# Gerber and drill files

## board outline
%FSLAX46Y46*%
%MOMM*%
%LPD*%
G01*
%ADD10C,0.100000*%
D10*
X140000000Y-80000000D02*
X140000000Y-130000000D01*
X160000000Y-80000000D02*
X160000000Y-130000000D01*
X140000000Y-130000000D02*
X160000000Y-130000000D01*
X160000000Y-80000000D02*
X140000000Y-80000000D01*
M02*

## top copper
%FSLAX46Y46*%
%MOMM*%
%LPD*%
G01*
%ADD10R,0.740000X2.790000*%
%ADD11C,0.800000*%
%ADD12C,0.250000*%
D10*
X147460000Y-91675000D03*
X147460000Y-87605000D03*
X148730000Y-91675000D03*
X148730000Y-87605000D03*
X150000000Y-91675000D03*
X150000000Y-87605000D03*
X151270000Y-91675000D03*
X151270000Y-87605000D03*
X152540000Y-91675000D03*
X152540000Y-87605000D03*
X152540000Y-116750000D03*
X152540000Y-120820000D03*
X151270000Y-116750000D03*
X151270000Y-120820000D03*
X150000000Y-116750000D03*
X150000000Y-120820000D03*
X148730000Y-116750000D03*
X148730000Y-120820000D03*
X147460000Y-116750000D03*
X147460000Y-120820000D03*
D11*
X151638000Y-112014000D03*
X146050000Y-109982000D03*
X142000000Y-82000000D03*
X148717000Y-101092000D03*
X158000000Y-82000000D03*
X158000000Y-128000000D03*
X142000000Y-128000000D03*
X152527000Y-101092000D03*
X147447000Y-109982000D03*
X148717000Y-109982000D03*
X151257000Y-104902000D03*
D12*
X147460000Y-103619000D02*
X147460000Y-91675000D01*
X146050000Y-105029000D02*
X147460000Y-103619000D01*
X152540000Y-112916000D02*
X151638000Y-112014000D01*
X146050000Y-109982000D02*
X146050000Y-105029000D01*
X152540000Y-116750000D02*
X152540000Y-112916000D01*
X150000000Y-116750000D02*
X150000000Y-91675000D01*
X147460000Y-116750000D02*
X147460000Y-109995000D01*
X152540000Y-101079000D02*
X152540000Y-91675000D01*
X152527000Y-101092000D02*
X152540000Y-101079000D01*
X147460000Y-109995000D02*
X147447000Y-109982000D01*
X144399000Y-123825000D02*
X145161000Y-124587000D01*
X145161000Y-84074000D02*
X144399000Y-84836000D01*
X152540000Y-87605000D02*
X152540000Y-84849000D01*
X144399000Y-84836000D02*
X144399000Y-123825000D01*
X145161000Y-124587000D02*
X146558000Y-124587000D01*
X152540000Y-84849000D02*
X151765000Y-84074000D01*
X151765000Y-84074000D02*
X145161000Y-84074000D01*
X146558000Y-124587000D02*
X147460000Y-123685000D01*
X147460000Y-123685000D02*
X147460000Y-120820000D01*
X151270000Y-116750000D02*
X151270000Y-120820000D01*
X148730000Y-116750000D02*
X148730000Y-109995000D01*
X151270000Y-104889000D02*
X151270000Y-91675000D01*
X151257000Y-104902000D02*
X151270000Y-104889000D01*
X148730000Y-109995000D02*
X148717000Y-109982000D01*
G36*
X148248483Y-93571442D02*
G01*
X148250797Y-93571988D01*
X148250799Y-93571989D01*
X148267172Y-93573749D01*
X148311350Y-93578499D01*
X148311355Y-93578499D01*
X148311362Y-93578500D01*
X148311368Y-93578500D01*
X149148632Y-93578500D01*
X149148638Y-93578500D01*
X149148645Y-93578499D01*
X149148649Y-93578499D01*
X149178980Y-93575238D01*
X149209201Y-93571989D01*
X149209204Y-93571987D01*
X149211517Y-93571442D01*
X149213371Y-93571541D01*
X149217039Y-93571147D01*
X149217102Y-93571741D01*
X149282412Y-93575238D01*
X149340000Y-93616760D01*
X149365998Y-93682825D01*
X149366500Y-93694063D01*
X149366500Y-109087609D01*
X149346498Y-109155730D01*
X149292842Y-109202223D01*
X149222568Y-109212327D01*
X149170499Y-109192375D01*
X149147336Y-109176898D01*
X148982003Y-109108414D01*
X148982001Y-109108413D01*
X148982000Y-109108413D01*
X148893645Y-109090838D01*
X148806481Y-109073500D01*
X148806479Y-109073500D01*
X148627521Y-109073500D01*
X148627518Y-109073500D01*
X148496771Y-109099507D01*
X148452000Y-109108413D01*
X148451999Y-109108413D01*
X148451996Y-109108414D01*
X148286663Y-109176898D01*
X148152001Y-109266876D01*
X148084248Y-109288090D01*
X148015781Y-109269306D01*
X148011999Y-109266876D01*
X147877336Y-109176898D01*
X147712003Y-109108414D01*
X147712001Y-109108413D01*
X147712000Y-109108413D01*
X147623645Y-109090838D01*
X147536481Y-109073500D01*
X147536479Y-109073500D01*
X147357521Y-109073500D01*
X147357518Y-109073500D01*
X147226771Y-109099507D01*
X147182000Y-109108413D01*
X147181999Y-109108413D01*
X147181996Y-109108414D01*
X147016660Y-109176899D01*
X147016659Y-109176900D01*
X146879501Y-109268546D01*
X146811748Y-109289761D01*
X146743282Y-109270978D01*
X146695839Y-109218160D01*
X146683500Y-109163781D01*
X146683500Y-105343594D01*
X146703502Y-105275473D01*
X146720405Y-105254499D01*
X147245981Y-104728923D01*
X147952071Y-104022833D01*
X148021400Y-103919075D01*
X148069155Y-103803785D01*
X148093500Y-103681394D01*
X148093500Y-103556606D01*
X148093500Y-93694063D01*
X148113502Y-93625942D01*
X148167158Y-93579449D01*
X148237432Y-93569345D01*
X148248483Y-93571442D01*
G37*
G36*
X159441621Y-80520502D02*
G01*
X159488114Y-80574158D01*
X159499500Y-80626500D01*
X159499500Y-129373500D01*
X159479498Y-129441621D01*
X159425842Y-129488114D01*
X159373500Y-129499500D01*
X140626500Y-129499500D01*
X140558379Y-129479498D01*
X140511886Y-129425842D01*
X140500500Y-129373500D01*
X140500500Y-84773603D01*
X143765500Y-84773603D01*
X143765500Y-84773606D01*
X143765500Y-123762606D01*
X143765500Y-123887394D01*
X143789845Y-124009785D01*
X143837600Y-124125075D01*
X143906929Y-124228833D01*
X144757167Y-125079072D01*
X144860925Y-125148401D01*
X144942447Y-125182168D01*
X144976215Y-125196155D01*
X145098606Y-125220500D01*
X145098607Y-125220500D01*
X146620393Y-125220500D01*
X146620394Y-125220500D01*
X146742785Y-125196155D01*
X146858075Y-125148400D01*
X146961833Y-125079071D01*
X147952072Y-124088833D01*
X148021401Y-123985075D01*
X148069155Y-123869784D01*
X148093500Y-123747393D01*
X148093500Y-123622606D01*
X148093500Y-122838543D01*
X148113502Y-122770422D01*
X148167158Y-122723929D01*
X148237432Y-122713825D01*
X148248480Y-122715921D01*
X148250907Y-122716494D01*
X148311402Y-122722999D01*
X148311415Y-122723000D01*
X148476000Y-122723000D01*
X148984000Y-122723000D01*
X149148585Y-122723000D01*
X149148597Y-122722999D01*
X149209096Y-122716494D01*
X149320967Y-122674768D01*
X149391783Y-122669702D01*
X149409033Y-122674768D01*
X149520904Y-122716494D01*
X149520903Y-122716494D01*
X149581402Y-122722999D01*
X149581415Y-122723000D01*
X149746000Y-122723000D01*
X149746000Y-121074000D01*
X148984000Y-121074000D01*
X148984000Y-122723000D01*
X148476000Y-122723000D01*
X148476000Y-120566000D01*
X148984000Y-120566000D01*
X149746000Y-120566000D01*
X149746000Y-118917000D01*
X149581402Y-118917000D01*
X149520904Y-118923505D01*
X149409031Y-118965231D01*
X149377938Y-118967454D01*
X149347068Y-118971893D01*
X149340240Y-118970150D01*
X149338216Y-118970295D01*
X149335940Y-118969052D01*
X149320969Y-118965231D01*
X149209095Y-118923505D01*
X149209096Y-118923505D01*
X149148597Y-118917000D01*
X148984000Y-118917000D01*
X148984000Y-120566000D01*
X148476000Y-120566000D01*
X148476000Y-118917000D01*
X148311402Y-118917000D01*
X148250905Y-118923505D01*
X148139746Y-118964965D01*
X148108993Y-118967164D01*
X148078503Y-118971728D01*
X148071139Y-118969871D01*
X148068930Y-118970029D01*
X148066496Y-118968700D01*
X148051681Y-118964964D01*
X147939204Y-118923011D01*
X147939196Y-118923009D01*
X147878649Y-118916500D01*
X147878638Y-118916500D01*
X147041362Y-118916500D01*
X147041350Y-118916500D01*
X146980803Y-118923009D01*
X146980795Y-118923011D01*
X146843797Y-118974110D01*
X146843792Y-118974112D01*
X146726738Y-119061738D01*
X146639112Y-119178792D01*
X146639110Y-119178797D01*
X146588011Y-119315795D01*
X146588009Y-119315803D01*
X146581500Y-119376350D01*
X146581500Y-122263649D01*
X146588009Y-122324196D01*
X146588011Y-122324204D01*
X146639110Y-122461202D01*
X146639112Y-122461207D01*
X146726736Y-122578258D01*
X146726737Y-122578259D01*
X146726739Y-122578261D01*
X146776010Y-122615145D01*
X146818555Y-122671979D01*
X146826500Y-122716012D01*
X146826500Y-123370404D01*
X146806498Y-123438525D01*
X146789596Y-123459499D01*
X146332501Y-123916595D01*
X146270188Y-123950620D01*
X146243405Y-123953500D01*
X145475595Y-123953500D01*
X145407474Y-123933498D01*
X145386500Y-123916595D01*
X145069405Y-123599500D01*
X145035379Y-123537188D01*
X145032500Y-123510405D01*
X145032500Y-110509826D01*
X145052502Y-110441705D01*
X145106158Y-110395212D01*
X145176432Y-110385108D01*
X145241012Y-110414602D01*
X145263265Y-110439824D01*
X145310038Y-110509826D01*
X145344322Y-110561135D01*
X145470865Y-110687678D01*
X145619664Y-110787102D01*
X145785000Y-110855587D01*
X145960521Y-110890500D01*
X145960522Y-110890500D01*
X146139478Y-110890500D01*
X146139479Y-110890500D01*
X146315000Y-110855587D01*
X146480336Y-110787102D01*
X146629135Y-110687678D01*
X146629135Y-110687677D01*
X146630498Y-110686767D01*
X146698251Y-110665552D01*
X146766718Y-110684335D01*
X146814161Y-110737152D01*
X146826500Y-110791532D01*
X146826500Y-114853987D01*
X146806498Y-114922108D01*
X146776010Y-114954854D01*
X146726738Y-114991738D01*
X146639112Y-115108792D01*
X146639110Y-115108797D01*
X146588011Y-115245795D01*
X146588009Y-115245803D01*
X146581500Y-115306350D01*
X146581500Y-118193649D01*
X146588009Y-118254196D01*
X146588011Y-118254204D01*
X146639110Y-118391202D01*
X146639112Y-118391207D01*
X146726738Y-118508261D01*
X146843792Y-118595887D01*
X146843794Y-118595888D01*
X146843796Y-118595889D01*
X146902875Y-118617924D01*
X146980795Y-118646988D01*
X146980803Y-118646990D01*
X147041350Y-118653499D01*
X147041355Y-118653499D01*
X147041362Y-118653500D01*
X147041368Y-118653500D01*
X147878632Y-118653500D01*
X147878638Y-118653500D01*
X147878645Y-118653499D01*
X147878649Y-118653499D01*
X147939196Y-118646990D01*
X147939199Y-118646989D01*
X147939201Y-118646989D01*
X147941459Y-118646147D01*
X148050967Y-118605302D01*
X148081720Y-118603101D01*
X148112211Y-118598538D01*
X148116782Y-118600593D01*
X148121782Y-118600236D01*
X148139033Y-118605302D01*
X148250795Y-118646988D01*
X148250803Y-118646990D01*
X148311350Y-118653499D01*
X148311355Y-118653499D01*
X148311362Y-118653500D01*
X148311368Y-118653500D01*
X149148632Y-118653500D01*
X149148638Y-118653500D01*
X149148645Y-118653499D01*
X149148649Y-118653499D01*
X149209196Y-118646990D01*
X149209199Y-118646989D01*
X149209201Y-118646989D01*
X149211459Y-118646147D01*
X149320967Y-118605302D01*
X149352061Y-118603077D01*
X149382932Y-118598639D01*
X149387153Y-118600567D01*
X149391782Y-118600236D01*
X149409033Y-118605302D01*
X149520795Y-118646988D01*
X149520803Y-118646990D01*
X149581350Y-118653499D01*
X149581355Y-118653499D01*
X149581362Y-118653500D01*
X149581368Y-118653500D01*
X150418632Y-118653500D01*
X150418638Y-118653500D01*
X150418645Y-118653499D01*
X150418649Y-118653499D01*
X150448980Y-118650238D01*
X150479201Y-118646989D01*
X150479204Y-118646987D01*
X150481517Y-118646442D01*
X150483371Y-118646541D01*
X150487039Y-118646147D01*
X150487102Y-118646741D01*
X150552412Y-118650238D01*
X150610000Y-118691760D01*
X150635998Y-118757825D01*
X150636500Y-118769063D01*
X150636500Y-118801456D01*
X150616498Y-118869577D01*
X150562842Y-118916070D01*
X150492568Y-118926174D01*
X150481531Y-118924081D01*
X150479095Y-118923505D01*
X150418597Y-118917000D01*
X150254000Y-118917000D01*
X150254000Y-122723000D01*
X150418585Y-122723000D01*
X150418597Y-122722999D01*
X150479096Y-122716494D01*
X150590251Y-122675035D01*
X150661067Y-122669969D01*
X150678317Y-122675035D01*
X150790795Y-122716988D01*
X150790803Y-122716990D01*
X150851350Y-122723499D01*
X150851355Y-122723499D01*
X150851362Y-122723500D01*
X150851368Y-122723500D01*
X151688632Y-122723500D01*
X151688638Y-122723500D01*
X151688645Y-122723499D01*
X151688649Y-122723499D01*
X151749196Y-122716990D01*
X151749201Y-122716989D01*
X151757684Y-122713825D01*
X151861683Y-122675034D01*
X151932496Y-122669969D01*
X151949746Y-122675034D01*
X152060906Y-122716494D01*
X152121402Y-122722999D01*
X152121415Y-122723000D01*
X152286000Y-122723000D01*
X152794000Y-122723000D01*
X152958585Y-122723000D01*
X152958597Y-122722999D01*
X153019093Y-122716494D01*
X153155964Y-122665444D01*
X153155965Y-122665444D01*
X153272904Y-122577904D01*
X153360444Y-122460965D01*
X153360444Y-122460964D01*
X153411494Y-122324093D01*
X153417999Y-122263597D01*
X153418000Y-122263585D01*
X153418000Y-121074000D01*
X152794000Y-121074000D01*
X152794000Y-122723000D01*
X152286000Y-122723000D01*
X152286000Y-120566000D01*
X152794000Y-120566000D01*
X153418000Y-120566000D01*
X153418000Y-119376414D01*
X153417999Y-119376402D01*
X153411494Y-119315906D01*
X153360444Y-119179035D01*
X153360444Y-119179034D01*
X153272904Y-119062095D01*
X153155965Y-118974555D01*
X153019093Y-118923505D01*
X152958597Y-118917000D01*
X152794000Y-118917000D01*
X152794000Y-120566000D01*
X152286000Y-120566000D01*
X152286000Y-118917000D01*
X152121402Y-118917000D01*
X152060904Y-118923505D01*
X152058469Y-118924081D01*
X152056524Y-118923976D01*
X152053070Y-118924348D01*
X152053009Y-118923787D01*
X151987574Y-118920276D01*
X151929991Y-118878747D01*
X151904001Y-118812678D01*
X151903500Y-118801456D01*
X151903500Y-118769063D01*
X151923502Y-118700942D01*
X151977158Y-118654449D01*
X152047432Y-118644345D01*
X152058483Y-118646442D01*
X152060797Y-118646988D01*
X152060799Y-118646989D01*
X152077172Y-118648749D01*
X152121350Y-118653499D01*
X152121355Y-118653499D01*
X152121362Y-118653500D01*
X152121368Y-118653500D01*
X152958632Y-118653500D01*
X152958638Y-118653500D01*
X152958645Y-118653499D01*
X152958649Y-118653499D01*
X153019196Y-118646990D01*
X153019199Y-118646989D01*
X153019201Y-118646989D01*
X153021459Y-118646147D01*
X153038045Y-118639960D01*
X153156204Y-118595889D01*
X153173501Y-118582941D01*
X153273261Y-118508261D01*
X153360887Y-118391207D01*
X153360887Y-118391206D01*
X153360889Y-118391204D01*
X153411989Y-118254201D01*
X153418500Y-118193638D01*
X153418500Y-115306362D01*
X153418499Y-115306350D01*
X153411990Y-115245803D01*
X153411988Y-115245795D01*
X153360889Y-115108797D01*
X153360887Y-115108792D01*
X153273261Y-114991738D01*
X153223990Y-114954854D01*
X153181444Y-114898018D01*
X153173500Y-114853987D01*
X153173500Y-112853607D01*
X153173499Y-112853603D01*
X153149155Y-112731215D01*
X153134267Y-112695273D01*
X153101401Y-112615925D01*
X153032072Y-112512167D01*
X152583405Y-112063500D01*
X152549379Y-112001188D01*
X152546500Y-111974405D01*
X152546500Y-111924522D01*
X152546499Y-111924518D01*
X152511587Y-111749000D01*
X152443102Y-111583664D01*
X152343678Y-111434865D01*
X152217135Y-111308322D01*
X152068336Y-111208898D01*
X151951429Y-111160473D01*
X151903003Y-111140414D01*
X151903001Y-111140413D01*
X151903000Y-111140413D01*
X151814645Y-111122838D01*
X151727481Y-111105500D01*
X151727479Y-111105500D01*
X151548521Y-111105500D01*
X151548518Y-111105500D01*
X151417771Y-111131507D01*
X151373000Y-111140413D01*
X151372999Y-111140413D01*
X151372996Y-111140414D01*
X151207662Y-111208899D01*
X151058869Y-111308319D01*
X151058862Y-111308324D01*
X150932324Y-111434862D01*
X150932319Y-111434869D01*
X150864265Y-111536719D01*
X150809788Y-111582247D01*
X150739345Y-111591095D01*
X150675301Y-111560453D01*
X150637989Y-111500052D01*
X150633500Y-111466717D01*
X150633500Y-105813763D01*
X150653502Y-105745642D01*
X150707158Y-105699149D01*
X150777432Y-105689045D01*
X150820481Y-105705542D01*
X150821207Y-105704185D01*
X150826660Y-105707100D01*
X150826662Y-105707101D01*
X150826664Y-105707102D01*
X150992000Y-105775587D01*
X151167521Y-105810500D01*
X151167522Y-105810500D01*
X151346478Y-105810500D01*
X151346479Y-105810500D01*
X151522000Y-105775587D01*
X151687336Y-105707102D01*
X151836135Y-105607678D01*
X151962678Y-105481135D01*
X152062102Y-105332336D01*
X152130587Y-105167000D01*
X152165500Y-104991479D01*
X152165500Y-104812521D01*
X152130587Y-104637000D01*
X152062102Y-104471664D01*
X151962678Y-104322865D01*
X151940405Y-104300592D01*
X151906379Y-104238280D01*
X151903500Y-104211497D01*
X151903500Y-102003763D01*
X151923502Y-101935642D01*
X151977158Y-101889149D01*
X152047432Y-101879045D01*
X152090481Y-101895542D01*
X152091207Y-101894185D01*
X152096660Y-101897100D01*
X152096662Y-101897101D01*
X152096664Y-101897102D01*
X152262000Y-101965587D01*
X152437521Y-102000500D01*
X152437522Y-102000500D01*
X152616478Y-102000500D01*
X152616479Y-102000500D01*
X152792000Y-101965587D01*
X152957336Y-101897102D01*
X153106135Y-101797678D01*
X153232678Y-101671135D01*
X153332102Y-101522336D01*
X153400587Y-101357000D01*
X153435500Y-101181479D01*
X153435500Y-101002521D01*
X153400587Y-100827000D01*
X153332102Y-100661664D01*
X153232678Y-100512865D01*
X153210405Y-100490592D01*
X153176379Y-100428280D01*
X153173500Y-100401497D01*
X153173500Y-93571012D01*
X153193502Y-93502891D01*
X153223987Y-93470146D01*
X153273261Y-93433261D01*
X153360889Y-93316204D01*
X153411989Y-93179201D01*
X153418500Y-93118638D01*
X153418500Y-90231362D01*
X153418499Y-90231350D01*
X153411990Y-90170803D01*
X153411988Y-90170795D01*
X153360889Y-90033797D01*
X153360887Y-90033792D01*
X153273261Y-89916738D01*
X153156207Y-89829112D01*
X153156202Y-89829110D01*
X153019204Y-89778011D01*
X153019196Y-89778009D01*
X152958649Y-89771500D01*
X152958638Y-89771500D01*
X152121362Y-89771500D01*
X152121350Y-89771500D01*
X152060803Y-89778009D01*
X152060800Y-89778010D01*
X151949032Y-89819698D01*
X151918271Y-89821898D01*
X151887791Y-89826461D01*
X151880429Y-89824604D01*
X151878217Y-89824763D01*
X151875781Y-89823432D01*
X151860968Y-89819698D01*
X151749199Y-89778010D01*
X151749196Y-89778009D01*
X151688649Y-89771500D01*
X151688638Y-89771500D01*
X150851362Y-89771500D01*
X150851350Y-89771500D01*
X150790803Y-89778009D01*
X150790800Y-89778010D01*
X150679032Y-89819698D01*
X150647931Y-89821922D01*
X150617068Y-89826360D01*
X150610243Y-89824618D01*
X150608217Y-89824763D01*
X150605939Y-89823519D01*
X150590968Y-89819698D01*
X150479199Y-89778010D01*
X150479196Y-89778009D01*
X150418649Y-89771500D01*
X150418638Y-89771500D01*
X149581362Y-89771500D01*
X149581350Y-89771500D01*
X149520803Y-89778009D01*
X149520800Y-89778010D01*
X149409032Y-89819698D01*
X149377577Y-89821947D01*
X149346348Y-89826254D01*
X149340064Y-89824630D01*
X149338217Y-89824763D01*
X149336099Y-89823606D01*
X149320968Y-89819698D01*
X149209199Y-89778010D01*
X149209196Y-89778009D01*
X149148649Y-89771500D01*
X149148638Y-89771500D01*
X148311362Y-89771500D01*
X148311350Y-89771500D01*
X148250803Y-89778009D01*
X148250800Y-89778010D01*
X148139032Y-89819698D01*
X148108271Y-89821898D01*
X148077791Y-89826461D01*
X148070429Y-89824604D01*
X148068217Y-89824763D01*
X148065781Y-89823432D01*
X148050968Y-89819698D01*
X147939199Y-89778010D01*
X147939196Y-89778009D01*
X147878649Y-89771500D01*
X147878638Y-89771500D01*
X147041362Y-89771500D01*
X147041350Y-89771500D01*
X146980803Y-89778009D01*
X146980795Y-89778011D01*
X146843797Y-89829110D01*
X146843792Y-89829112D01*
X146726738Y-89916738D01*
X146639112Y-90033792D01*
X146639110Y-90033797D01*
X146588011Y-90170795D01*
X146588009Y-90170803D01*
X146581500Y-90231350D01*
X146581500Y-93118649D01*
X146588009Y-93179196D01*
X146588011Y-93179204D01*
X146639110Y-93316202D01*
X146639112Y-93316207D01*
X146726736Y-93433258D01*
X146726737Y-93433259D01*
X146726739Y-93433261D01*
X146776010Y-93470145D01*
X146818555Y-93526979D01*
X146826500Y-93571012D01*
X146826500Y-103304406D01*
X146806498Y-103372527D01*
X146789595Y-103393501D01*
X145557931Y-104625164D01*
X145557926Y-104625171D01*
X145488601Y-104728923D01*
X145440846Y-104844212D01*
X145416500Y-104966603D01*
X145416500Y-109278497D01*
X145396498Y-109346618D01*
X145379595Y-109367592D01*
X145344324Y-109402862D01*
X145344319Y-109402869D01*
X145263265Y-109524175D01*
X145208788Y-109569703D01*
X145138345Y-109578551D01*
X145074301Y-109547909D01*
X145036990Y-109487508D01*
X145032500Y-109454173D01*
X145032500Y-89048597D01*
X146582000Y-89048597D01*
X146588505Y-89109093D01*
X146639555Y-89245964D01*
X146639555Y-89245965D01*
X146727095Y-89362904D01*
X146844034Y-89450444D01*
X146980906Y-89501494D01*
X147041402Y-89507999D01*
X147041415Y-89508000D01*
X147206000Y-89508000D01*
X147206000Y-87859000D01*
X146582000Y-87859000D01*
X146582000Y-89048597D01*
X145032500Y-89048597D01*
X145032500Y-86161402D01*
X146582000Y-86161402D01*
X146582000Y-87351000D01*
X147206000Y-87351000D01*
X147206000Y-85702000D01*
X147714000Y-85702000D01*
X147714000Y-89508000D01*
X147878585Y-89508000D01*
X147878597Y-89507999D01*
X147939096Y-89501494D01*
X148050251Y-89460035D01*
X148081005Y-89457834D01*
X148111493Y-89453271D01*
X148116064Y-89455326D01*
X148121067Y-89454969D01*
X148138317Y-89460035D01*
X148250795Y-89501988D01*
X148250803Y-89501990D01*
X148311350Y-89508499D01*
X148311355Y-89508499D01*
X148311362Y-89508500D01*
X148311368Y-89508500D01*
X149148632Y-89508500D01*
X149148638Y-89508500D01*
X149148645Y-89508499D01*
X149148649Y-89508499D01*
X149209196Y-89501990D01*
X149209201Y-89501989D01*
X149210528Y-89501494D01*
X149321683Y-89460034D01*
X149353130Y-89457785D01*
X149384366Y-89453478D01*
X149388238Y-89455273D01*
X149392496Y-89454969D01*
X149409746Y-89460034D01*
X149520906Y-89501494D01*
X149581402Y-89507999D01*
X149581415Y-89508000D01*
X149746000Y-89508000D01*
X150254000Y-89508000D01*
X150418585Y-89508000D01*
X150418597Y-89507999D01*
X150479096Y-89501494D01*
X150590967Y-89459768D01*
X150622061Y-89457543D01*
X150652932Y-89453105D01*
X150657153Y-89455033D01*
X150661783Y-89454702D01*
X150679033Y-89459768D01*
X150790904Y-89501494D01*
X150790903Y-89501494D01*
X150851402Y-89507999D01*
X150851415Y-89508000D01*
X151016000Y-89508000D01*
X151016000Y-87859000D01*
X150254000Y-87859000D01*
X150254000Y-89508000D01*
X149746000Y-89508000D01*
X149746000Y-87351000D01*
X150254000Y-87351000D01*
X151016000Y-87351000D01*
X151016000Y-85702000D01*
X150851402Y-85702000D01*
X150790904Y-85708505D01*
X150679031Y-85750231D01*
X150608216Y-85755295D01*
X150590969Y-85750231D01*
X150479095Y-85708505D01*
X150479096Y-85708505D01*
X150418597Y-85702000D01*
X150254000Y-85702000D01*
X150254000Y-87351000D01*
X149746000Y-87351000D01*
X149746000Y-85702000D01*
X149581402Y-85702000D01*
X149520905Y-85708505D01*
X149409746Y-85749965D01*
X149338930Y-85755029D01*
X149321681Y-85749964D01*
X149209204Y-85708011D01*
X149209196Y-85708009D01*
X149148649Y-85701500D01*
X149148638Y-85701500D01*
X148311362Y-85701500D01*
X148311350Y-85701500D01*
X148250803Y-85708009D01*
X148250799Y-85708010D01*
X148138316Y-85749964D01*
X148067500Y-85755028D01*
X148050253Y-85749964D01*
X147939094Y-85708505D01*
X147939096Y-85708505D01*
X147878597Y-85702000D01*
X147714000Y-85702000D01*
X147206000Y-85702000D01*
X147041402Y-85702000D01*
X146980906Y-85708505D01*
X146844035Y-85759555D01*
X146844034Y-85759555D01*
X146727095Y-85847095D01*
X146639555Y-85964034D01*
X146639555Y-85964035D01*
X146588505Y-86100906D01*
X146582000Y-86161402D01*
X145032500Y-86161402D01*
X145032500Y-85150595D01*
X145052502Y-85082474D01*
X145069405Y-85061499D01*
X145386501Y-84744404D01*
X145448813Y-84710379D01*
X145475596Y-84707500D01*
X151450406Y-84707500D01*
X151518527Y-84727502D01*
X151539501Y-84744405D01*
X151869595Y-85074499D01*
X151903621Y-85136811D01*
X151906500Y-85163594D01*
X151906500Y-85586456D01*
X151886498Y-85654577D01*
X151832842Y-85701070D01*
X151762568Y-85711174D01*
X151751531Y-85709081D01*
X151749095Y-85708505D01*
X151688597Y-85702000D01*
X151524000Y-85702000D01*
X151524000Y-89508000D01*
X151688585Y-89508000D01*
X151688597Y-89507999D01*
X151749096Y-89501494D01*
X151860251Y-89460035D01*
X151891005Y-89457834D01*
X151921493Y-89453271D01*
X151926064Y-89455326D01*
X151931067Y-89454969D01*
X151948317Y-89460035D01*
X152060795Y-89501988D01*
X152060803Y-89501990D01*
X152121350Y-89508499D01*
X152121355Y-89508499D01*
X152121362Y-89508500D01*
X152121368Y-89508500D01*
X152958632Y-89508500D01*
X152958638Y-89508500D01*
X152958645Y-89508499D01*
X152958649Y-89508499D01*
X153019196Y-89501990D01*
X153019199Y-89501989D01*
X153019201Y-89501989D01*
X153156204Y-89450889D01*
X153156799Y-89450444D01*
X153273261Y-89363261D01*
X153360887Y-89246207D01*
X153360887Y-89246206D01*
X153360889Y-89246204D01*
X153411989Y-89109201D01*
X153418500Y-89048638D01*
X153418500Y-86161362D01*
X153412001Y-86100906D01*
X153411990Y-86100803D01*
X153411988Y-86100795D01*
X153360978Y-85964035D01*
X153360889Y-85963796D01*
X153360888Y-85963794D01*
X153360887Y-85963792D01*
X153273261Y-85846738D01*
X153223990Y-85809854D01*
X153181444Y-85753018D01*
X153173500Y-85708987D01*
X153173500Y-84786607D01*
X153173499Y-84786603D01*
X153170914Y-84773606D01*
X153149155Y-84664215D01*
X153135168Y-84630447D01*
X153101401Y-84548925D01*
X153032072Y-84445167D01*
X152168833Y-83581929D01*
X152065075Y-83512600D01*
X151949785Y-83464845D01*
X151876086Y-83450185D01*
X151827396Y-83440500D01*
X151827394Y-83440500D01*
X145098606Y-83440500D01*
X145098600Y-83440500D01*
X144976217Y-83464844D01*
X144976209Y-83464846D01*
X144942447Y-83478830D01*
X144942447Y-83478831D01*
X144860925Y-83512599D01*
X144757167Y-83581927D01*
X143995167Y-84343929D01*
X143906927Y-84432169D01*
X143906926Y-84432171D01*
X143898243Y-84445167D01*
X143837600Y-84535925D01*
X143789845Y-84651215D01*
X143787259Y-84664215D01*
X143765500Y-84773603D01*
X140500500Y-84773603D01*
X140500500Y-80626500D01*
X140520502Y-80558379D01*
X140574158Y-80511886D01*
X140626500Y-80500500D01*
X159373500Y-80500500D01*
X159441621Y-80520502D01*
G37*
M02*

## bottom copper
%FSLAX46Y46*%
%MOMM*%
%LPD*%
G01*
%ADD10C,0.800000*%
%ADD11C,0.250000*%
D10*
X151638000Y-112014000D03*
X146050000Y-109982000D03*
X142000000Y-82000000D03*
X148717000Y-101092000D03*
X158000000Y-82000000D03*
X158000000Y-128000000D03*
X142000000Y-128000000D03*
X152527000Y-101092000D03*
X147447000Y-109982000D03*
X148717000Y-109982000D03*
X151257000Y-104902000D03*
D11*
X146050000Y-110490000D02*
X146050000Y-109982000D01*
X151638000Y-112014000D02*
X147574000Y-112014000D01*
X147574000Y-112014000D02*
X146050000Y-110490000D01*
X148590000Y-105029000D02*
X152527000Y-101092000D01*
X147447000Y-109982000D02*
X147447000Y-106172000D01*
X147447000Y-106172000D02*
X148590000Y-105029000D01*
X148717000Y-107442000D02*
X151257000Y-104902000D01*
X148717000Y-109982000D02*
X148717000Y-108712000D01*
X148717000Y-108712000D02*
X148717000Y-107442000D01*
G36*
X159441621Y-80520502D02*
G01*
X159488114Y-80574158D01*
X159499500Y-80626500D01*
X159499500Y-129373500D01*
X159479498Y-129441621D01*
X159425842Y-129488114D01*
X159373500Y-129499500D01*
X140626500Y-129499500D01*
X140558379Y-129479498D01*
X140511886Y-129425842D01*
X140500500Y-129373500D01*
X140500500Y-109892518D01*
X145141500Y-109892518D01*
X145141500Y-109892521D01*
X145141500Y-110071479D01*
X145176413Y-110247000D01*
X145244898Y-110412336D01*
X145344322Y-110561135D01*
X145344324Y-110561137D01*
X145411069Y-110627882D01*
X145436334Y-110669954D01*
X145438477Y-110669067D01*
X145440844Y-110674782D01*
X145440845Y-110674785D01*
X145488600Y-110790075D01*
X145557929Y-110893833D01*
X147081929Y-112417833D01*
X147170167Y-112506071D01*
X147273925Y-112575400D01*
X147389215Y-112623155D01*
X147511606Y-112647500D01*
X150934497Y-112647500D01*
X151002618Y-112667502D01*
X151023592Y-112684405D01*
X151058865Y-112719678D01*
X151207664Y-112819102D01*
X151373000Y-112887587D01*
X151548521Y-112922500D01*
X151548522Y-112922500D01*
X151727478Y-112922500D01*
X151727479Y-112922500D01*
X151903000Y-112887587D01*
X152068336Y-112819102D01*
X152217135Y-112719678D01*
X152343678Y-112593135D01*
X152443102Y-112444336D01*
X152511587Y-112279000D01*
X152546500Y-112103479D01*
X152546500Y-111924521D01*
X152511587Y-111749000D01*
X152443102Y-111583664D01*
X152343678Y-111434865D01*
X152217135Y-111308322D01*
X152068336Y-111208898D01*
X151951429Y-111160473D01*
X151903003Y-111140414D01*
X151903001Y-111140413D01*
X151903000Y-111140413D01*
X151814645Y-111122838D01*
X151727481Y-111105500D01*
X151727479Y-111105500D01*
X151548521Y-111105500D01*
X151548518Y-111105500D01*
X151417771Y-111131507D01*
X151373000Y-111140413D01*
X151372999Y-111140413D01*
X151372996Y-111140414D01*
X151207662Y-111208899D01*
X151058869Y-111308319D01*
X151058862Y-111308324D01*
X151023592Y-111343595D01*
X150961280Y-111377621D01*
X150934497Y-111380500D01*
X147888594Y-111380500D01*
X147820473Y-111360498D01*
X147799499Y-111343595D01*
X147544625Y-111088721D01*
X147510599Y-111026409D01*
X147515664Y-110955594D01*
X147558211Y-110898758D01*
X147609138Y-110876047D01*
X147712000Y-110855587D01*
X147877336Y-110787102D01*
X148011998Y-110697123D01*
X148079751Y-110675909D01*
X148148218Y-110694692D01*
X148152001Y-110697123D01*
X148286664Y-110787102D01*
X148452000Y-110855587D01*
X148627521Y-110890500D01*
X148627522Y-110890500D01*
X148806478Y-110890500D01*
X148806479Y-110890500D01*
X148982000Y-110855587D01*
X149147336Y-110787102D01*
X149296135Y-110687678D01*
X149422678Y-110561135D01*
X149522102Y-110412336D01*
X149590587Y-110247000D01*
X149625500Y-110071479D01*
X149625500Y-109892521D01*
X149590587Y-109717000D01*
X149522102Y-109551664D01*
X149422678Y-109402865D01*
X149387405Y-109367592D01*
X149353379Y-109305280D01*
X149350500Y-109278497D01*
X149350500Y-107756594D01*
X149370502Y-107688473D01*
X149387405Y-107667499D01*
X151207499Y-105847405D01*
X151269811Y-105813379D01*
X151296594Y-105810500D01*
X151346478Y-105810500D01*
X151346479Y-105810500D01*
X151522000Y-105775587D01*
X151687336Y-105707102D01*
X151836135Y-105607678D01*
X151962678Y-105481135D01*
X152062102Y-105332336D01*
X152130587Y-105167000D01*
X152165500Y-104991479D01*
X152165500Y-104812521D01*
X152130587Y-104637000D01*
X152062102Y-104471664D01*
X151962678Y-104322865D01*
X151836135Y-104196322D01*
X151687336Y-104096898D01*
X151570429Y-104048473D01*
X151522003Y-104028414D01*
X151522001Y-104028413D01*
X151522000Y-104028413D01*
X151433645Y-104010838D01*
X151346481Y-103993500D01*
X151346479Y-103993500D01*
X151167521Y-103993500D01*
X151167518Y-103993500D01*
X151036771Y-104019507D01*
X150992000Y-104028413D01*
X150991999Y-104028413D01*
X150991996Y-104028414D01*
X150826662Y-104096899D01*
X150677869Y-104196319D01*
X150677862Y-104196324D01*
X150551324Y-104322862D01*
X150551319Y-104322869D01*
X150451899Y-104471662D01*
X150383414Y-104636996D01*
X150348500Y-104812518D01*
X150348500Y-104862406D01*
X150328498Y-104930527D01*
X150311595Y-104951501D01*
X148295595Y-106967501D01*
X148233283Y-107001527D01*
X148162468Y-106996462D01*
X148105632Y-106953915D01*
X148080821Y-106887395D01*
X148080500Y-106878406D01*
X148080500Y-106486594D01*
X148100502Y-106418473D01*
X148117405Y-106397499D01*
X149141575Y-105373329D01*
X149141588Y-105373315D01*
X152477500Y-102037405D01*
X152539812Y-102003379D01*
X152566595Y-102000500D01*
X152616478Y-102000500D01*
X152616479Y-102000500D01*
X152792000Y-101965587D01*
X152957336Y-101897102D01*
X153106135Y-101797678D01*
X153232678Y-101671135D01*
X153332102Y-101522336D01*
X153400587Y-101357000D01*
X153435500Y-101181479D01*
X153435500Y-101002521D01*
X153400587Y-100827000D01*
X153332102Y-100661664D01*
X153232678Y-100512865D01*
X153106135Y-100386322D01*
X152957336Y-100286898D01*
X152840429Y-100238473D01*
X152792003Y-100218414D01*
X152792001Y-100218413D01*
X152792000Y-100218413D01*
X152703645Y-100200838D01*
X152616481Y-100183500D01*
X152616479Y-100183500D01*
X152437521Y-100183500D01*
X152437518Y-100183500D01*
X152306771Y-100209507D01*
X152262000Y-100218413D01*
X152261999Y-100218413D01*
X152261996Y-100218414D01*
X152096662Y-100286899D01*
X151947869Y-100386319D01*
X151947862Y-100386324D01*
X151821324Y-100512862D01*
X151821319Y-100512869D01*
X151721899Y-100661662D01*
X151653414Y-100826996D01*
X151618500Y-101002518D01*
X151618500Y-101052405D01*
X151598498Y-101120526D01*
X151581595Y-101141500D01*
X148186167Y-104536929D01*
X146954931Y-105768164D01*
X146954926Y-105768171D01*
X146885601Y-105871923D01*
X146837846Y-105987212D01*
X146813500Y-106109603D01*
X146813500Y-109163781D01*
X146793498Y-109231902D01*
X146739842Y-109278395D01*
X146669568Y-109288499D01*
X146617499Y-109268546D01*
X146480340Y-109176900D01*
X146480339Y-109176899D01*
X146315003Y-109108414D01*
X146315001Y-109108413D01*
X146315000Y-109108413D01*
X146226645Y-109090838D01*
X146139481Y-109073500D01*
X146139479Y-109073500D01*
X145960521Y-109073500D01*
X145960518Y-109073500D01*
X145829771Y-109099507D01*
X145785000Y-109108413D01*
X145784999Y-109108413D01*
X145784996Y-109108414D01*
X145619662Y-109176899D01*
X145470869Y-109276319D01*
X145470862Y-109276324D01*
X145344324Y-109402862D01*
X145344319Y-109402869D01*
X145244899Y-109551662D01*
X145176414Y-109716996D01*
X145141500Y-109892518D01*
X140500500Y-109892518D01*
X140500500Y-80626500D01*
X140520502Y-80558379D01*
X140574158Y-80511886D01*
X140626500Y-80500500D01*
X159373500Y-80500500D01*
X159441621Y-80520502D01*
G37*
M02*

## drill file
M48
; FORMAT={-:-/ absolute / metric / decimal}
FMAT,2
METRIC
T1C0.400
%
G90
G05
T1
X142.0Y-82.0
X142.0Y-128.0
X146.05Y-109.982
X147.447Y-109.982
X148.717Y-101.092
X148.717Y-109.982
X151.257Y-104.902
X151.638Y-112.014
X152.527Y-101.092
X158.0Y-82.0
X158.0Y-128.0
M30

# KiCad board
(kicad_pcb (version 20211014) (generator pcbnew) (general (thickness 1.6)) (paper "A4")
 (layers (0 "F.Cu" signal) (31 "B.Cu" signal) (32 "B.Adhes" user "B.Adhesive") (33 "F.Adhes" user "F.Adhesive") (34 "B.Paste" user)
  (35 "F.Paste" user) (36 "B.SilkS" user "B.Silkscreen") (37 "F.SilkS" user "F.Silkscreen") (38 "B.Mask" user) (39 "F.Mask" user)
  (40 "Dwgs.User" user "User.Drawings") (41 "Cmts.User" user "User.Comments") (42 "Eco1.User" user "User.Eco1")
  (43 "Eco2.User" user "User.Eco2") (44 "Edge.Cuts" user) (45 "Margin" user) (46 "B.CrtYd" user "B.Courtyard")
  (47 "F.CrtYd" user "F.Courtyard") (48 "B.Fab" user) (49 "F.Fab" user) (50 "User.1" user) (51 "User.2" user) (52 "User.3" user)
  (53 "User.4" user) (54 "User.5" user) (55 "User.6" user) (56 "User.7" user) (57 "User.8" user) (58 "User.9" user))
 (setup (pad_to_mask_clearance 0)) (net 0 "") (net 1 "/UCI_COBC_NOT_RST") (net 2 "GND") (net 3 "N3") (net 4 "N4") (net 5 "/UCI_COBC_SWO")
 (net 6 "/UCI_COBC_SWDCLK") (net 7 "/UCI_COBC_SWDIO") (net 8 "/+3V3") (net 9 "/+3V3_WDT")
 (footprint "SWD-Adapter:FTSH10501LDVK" (layer "F.Cu") (at 150 91.675)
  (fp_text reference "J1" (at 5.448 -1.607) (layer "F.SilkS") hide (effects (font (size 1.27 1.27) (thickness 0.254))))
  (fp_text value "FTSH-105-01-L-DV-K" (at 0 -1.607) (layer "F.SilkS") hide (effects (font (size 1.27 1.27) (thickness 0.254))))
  (pad "1" smd rect (at -2.54 0) (size 0.74 2.79) (layers "F.Cu" "F.Paste" "F.Mask") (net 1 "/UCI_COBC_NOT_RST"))
  (pad "2" smd rect (at -2.54 -4.07) (size 0.74 2.79) (layers "F.Cu" "F.Paste" "F.Mask") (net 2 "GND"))
  (pad "3" smd rect (at -1.27 0) (size 0.74 2.79) (layers "F.Cu" "F.Paste" "F.Mask") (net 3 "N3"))
  (pad "4" smd rect (at -1.27 -4.07) (size 0.74 2.79) (layers "F.Cu" "F.Paste" "F.Mask") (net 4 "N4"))
  (pad "5" smd rect (at 0 0) (size 0.74 2.79) (layers "F.Cu" "F.Paste" "F.Mask") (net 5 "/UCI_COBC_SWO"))
  (pad "6" smd rect (at 0 -4.07) (size 0.74 2.79) (layers "F.Cu" "F.Paste" "F.Mask") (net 2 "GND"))
  (pad "7" smd rect (at 1.27 0) (size 0.74 2.79) (layers "F.Cu" "F.Paste" "F.Mask") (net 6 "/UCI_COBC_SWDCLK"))
  (pad "8" smd rect (at 1.27 -4.07) (size 0.74 2.79) (layers "F.Cu" "F.Paste" "F.Mask") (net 2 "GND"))
  (pad "9" smd rect (at 2.54 0) (size 0.74 2.79) (layers "F.Cu" "F.Paste" "F.Mask") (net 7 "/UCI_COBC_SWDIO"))
  (pad "10" smd rect (at 2.54 -4.07) (size 0.74 2.79) (layers "F.Cu" "F.Paste" "F.Mask") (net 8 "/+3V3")))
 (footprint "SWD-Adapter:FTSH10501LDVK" (layer "F.Cu") (at 150 116.75 180)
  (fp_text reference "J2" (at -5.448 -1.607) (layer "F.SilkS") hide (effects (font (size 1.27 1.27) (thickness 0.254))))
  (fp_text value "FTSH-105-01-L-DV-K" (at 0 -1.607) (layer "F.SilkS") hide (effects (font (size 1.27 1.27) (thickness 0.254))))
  (pad "1" smd rect (at -2.54 0 180) (size 0.74 2.79) (layers "F.Cu" "F.Paste" "F.Mask") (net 1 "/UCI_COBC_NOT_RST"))
  (pad "2" smd rect (at -2.54 -4.07 180) (size 0.74 2.79) (layers "F.Cu" "F.Paste" "F.Mask") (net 2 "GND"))
  (pad "3" smd rect (at -1.27 0 180) (size 0.74 2.79) (layers "F.Cu" "F.Paste" "F.Mask") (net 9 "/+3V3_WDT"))
  (pad "4" smd rect (at -1.27 -4.07 180) (size 0.74 2.79) (layers "F.Cu" "F.Paste" "F.Mask") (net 9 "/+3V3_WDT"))
  (pad "5" smd rect (at 0 0 180) (size 0.74 2.79) (layers "F.Cu" "F.Paste" "F.Mask") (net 5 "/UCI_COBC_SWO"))
  (pad "6" smd rect (at 0 -4.07 180) (size 0.74 2.79) (layers "F.Cu" "F.Paste" "F.Mask") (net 2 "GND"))
  (pad "7" smd rect (at 1.27 0 180) (size 0.74 2.79) (layers "F.Cu" "F.Paste" "F.Mask") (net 6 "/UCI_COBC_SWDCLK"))
  (pad "8" smd rect (at 1.27 -4.07 180) (size 0.74 2.79) (layers "F.Cu" "F.Paste" "F.Mask") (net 2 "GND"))
  (pad "9" smd rect (at 2.54 0 180) (size 0.74 2.79) (layers "F.Cu" "F.Paste" "F.Mask") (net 7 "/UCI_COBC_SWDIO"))
  (pad "10" smd rect (at 2.54 -4.07 180) (size 0.74 2.79) (layers "F.Cu" "F.Paste" "F.Mask") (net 8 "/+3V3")))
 (gr_line (start 140 80) (end 140 130) (layer "Edge.Cuts") (width 0.1))
 (gr_line (start 160 80) (end 160 130) (layer "Edge.Cuts") (width 0.1))
 (gr_line (start 140 130) (end 160 130) (layer "Edge.Cuts") (width 0.1))
 (gr_line (start 160 80) (end 140 80) (layer "Edge.Cuts") (width 0.1))
 (segment (start 147.46 103.619) (end 147.46 91.675) (width 0.25) (layer "F.Cu") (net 1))
 (segment (start 146.05 105.029) (end 147.46 103.619) (width 0.25) (layer "F.Cu") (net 1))
 (segment (start 152.54 112.916) (end 151.638 112.014) (width 0.25) (layer "F.Cu") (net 1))
 (segment (start 146.05 109.982) (end 146.05 105.029) (width 0.25) (layer "F.Cu") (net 1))
 (segment (start 152.54 116.75) (end 152.54 112.916) (width 0.25) (layer "F.Cu") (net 1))
 (via (at 151.638 112.014) (size 0.8) (drill 0.4) (layers "F.Cu" "B.Cu") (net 1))
 (via (at 146.05 109.982) (size 0.8) (drill 0.4) (layers "F.Cu" "B.Cu") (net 1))
 (segment (start 146.05 110.49) (end 146.05 109.982) (width 0.25) (layer "B.Cu") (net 1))
 (segment (start 151.638 112.014) (end 147.574 112.014) (width 0.25) (layer "B.Cu") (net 1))
 (segment (start 147.574 112.014) (end 146.05 110.49) (width 0.25) (layer "B.Cu") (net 1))
 (via (at 142 82) (size 0.8) (drill 0.4) (layers "F.Cu" "B.Cu") (free) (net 2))
 (via (at 148.717 101.092) (size 0.8) (drill 0.4) (layers "F.Cu" "B.Cu") (free) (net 2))
 (via (at 158 82) (size 0.8) (drill 0.4) (layers "F.Cu" "B.Cu") (free) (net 2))
 (via (at 158 128) (size 0.8) (drill 0.4) (layers "F.Cu" "B.Cu") (free) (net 2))
 (via (at 142 128) (size 0.8) (drill 0.4) (layers "F.Cu" "B.Cu") (free) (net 2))
 (segment (start 150 116.75) (end 150 91.675) (width 0.25) (layer "F.Cu") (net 5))
 (segment (start 147.46 116.75) (end 147.46 109.995) (width 0.25) (layer "F.Cu") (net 7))
 (segment (start 152.54 101.079) (end 152.54 91.675) (width 0.25) (layer "F.Cu") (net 7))
 (segment (start 152.527 101.092) (end 152.54 101.079) (width 0.25) (layer "F.Cu") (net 7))
 (segment (start 147.46 109.995) (end 147.447 109.982) (width 0.25) (layer "F.Cu") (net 7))
 (via (at 152.527 101.092) (size 0.8) (drill 0.4) (layers "F.Cu" "B.Cu") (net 7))
 (via (at 147.447 109.982) (size 0.8) (drill 0.4) (layers "F.Cu" "B.Cu") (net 7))
 (segment (start 148.59 105.029) (end 152.527 101.092) (width 0.25) (layer "B.Cu") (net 7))
 (segment (start 147.447 109.982) (end 147.447 106.172) (width 0.25) (layer "B.Cu") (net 7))
 (segment (start 147.447 106.172) (end 148.59 105.029) (width 0.25) (layer "B.Cu") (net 7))
 (segment (start 144.399 123.825) (end 145.161 124.587) (width 0.25) (layer "F.Cu") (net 8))
 (segment (start 145.161 84.074) (end 144.399 84.836) (width 0.25) (layer "F.Cu") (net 8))
 (segment (start 152.54 87.605) (end 152.54 84.849) (width 0.25) (layer "F.Cu") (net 8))
 (segment (start 144.399 84.836) (end 144.399 123.825) (width 0.25) (layer "F.Cu") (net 8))
 (segment (start 145.161 124.587) (end 146.558 124.587) (width 0.25) (layer "F.Cu") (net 8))
 (segment (start 152.54 84.849) (end 151.765 84.074) (width 0.25) (layer "F.Cu") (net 8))
 (segment (start 151.765 84.074) (end 145.161 84.074) (width 0.25) (layer "F.Cu") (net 8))
 (segment (start 146.558 124.587) (end 147.46 123.685) (width 0.25) (layer "F.Cu") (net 8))
 (segment (start 147.46 123.685) (end 147.46 120.82) (width 0.25) (layer "F.Cu") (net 8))
 (segment (start 151.27 116.75) (end 151.27 120.82) (width 0.25) (layer "F.Cu") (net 9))
 (segment (start 148.73 116.75) (end 148.73 109.995) (width 0.25) (layer "F.Cu") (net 6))
 (segment (start 151.27 104.889) (end 151.27 91.675) (width 0.25) (layer "F.Cu") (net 6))
 (segment (start 151.257 104.902) (end 151.27 104.889) (width 0.25) (layer "F.Cu") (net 6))
 (segment (start 148.73 109.995) (end 148.717 109.982) (width 0.25) (layer "F.Cu") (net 6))
 (via (at 148.717 109.982) (size 0.8) (drill 0.4) (layers "F.Cu" "B.Cu") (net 6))
 (via (at 151.257 104.902) (size 0.8) (drill 0.4) (layers "F.Cu" "B.Cu") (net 6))
 (segment (start 148.717 107.442) (end 151.257 104.902) (width 0.25) (layer "B.Cu") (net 6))
 (segment (start 148.717 109.982) (end 148.717 108.712) (width 0.25) (layer "B.Cu") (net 6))
 (segment (start 148.717 108.712) (end 148.717 107.442) (width 0.25) (layer "B.Cu") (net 6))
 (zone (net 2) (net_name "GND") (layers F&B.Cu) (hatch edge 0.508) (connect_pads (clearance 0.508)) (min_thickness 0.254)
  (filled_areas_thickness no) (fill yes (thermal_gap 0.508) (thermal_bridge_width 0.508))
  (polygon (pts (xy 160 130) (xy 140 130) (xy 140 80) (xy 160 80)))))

